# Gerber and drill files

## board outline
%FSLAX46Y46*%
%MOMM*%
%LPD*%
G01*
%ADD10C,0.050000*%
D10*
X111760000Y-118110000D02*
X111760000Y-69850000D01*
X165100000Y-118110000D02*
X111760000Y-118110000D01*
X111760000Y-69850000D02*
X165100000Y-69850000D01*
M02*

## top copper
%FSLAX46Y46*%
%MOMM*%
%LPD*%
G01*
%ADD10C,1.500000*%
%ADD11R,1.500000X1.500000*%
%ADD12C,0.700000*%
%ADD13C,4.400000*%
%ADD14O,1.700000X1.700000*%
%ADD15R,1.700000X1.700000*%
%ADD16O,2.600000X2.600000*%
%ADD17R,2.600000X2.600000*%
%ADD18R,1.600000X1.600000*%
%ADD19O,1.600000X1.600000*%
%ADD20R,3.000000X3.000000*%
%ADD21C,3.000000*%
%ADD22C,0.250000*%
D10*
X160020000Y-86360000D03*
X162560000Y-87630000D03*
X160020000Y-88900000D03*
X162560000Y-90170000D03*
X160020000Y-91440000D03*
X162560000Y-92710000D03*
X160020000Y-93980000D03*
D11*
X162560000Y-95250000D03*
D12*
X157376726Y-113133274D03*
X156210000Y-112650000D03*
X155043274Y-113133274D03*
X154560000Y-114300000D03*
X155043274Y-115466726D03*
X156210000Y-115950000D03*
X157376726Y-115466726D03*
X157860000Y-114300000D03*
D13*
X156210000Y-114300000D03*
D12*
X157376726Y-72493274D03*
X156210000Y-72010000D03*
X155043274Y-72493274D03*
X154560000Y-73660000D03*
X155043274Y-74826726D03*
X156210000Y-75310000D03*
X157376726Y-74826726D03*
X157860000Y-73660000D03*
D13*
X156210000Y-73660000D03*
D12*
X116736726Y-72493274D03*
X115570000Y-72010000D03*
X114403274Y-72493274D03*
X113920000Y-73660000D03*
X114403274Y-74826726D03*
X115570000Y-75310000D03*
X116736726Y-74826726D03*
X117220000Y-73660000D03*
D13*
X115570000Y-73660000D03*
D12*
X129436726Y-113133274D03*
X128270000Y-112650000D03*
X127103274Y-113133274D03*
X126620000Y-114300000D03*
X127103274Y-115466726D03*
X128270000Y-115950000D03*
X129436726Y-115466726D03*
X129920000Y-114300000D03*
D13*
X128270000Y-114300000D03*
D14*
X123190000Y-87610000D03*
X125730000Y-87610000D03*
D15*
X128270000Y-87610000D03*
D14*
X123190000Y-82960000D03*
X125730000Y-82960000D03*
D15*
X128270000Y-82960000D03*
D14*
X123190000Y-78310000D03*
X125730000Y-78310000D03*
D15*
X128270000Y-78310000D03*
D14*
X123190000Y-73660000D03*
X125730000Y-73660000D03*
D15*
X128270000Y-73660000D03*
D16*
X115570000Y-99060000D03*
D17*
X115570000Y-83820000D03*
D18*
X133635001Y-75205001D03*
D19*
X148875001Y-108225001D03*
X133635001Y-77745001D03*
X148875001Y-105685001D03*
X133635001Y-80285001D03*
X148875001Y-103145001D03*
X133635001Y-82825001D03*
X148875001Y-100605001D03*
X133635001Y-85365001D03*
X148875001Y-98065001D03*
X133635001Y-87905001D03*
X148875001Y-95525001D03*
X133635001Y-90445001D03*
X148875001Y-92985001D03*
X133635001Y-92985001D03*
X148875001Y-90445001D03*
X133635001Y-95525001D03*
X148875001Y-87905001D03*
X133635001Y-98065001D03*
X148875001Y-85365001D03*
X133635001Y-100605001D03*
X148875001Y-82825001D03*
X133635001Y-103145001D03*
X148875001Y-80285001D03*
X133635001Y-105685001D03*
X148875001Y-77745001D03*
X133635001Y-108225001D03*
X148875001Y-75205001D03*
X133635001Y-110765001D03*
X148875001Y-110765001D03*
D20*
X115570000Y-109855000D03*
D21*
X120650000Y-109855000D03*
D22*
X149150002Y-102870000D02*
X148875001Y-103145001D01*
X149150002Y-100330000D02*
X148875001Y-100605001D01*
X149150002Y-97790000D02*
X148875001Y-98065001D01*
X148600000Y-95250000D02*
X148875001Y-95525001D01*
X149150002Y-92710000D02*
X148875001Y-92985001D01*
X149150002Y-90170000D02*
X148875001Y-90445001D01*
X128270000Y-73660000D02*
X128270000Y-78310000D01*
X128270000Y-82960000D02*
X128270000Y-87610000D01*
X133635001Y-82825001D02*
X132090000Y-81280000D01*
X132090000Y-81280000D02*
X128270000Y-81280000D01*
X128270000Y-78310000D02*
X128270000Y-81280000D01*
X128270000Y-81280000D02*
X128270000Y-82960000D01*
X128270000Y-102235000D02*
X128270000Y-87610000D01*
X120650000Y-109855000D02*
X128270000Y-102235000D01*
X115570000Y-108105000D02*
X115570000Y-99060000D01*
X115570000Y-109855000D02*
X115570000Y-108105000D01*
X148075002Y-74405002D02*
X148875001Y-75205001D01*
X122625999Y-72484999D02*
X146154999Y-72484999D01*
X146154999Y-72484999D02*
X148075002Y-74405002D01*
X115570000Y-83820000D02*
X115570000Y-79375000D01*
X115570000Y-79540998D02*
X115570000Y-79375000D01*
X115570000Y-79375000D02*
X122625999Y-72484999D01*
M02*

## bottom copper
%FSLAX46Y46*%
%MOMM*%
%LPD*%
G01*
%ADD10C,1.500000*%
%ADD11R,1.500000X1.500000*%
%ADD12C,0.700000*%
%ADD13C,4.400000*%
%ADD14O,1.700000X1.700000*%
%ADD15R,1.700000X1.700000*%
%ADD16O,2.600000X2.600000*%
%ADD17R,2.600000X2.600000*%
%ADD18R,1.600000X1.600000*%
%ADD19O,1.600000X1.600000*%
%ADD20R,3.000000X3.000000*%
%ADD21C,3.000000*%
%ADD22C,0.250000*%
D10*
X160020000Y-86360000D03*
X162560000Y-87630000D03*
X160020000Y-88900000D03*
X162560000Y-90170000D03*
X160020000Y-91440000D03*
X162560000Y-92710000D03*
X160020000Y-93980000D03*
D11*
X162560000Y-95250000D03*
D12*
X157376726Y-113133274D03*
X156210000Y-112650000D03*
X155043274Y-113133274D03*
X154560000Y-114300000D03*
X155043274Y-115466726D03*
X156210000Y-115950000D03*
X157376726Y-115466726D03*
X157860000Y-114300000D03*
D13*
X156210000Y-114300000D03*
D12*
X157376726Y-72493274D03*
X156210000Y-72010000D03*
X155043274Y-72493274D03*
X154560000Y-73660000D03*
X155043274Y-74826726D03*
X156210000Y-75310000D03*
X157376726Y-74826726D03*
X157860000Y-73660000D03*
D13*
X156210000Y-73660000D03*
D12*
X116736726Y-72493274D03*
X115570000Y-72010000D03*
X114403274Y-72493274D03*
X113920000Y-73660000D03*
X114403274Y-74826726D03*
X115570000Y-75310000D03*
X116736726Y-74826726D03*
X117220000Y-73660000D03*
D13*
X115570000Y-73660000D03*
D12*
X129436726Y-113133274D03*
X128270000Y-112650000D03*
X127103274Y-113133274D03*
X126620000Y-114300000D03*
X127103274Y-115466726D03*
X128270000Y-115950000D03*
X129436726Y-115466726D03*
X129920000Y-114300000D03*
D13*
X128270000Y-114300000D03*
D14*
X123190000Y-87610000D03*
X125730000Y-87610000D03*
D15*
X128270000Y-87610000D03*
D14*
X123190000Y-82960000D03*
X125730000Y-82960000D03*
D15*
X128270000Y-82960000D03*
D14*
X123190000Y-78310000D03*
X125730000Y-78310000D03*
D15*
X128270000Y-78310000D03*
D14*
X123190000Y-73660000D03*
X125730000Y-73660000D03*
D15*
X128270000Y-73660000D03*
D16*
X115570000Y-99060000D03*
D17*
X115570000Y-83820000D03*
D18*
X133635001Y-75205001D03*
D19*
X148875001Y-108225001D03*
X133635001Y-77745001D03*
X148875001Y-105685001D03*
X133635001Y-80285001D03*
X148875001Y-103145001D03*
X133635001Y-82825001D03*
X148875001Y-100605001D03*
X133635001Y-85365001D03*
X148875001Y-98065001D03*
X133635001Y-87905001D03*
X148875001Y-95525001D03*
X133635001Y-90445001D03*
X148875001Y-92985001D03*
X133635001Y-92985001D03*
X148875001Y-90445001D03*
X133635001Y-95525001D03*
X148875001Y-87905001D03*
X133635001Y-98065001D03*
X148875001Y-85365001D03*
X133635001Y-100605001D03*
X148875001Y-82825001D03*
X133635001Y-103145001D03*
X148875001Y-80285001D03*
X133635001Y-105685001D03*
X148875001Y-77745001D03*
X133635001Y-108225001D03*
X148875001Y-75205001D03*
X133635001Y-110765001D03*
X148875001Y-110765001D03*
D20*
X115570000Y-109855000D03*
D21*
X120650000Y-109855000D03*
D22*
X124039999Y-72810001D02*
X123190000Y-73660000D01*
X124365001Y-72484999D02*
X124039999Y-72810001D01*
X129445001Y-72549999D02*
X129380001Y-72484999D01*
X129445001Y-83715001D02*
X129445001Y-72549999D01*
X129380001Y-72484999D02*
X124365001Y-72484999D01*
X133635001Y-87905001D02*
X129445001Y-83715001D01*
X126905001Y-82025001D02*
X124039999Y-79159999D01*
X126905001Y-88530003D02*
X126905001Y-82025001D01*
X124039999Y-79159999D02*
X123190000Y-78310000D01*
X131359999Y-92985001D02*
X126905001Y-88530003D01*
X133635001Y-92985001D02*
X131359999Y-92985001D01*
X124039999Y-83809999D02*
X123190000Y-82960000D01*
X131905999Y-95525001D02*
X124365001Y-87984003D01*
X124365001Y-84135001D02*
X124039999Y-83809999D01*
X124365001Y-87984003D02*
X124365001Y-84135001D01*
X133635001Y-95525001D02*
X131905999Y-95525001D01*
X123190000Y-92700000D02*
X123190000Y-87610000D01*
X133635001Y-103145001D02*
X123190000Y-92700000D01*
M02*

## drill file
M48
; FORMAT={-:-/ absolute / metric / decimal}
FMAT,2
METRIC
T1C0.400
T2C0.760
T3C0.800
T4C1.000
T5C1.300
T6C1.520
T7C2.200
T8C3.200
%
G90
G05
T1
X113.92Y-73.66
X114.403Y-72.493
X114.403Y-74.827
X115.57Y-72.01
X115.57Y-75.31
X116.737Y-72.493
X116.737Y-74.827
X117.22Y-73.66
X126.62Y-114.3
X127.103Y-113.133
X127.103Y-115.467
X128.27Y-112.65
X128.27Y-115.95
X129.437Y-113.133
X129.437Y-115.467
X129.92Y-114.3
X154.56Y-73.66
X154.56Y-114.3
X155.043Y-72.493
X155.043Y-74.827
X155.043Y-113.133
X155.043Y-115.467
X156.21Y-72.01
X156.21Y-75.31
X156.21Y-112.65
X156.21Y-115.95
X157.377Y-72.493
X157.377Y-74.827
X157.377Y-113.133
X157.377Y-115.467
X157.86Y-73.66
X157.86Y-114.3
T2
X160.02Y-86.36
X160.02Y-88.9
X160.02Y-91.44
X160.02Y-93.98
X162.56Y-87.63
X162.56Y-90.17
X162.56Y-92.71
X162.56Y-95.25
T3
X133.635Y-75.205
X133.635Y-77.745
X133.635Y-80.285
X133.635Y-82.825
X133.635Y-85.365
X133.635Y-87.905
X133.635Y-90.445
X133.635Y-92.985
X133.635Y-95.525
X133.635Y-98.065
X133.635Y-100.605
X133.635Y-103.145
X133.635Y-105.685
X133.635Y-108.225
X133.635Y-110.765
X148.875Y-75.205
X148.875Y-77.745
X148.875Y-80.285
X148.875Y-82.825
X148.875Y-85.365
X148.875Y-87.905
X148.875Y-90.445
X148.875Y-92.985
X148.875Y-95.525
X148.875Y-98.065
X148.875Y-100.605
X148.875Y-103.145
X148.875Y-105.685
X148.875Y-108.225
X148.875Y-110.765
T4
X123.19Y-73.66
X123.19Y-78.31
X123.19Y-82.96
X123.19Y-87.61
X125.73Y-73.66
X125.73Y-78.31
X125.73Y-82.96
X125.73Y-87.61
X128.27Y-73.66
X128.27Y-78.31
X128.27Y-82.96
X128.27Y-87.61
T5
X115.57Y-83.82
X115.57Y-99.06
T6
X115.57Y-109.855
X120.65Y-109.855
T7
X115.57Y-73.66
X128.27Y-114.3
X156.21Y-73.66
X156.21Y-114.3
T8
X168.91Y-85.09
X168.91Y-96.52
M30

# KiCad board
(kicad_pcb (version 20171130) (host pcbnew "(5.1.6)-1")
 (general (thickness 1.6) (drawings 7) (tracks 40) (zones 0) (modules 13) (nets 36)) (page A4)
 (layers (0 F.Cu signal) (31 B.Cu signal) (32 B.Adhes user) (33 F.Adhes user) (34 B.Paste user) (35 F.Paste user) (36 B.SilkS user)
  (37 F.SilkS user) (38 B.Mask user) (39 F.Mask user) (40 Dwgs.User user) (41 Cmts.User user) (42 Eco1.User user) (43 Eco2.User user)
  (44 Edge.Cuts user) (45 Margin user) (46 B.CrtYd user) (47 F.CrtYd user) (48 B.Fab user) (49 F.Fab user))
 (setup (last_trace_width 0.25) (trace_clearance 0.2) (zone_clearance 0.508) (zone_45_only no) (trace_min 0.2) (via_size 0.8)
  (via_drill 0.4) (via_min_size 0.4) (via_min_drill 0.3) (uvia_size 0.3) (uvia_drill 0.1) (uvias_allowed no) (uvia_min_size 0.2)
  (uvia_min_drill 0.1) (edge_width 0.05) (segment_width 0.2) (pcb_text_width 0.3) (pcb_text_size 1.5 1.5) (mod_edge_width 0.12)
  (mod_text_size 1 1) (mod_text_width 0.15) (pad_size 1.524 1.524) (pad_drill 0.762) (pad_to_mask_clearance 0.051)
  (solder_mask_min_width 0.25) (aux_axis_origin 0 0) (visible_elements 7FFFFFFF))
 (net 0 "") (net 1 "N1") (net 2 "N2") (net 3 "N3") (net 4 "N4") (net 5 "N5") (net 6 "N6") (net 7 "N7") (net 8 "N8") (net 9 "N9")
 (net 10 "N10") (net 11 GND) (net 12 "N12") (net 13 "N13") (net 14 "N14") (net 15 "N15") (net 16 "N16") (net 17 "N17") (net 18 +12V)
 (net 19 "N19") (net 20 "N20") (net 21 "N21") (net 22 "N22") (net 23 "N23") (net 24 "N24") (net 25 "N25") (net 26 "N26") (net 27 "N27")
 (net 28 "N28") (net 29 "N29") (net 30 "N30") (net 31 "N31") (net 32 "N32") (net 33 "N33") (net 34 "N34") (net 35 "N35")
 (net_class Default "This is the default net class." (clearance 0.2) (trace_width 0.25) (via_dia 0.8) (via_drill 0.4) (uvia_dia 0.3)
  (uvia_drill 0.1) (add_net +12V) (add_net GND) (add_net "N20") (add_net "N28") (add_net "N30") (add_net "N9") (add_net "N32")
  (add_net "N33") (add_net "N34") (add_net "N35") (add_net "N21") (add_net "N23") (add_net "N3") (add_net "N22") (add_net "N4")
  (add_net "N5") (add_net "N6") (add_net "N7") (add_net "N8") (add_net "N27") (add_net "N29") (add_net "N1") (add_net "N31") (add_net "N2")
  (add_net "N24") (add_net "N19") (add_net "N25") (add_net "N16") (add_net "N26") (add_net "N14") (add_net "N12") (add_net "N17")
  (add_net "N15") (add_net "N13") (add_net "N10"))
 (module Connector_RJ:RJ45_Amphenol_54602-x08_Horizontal (layer F.Cu) (at 162.56 95.25 90)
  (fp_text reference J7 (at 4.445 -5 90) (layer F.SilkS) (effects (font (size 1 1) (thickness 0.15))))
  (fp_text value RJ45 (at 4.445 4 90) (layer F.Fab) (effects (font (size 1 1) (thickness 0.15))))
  (pad 8 thru_hole circle (at 8.89 -2.54 90) (size 1.5 1.5) (drill 0.76) (layers *.Cu *.Mask) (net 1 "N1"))
  (pad 7 thru_hole circle (at 7.62 0 90) (size 1.5 1.5) (drill 0.76) (layers *.Cu *.Mask) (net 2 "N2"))
  (pad 6 thru_hole circle (at 6.35 -2.54 90) (size 1.5 1.5) (drill 0.76) (layers *.Cu *.Mask) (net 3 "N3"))
  (pad 5 thru_hole circle (at 5.08 0 90) (size 1.5 1.5) (drill 0.76) (layers *.Cu *.Mask) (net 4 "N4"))
  (pad 4 thru_hole circle (at 3.81 -2.54 90) (size 1.5 1.5) (drill 0.76) (layers *.Cu *.Mask) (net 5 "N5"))
  (pad 3 thru_hole circle (at 2.54 0 90) (size 1.5 1.5) (drill 0.76) (layers *.Cu *.Mask) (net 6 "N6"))
  (pad 2 thru_hole circle (at 1.27 -2.54 90) (size 1.5 1.5) (drill 0.76) (layers *.Cu *.Mask) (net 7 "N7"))
  (pad 1 thru_hole rect (at 0 0 90) (size 1.5 1.5) (drill 0.76) (layers *.Cu *.Mask) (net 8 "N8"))
  (pad "" np_thru_hole circle (at -1.27 6.35 90) (size 3.2 3.2) (drill 3.2) (layers *.Cu *.Mask))
  (pad "" np_thru_hole circle (at 10.16 6.35 90) (size 3.2 3.2) (drill 3.2) (layers *.Cu *.Mask)))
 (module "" (layer B.Cu) (at 140.97 92.71 270)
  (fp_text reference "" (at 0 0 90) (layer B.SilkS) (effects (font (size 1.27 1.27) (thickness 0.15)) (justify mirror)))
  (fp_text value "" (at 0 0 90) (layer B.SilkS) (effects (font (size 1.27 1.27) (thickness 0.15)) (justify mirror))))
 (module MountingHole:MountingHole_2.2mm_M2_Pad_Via (layer F.Cu) (at 156.21 114.3)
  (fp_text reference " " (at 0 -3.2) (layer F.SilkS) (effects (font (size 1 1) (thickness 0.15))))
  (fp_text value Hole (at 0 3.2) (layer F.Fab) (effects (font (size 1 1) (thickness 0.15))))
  (pad 1 thru_hole circle (at 1.166726 -1.166726) (size 0.7 0.7) (drill 0.4) (layers *.Cu *.Mask))
  (pad 1 thru_hole circle (at 0 -1.65) (size 0.7 0.7) (drill 0.4) (layers *.Cu *.Mask))
  (pad 1 thru_hole circle (at -1.166726 -1.166726) (size 0.7 0.7) (drill 0.4) (layers *.Cu *.Mask))
  (pad 1 thru_hole circle (at -1.65 0) (size 0.7 0.7) (drill 0.4) (layers *.Cu *.Mask))
  (pad 1 thru_hole circle (at -1.166726 1.166726) (size 0.7 0.7) (drill 0.4) (layers *.Cu *.Mask))
  (pad 1 thru_hole circle (at 0 1.65) (size 0.7 0.7) (drill 0.4) (layers *.Cu *.Mask))
  (pad 1 thru_hole circle (at 1.166726 1.166726) (size 0.7 0.7) (drill 0.4) (layers *.Cu *.Mask))
  (pad 1 thru_hole circle (at 1.65 0) (size 0.7 0.7) (drill 0.4) (layers *.Cu *.Mask))
  (pad 1 thru_hole circle (at 0 0) (size 4.4 4.4) (drill 2.2) (layers *.Cu *.Mask)))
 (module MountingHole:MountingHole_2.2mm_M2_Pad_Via (layer F.Cu) (at 156.21 73.66)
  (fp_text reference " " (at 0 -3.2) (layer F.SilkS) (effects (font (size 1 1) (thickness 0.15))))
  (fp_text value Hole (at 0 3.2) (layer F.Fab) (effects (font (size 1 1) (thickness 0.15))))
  (pad 1 thru_hole circle (at 1.166726 -1.166726) (size 0.7 0.7) (drill 0.4) (layers *.Cu *.Mask))
  (pad 1 thru_hole circle (at 0 -1.65) (size 0.7 0.7) (drill 0.4) (layers *.Cu *.Mask))
  (pad 1 thru_hole circle (at -1.166726 -1.166726) (size 0.7 0.7) (drill 0.4) (layers *.Cu *.Mask))
  (pad 1 thru_hole circle (at -1.65 0) (size 0.7 0.7) (drill 0.4) (layers *.Cu *.Mask))
  (pad 1 thru_hole circle (at -1.166726 1.166726) (size 0.7 0.7) (drill 0.4) (layers *.Cu *.Mask))
  (pad 1 thru_hole circle (at 0 1.65) (size 0.7 0.7) (drill 0.4) (layers *.Cu *.Mask))
  (pad 1 thru_hole circle (at 1.166726 1.166726) (size 0.7 0.7) (drill 0.4) (layers *.Cu *.Mask))
  (pad 1 thru_hole circle (at 1.65 0) (size 0.7 0.7) (drill 0.4) (layers *.Cu *.Mask))
  (pad 1 thru_hole circle (at 0 0) (size 4.4 4.4) (drill 2.2) (layers *.Cu *.Mask)))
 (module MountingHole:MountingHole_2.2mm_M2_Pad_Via (layer F.Cu) (at 115.57 73.66)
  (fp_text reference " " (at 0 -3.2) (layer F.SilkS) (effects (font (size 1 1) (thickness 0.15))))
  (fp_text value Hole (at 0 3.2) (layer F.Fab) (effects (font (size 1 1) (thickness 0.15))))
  (pad 1 thru_hole circle (at 1.166726 -1.166726) (size 0.7 0.7) (drill 0.4) (layers *.Cu *.Mask))
  (pad 1 thru_hole circle (at 0 -1.65) (size 0.7 0.7) (drill 0.4) (layers *.Cu *.Mask))
  (pad 1 thru_hole circle (at -1.166726 -1.166726) (size 0.7 0.7) (drill 0.4) (layers *.Cu *.Mask))
  (pad 1 thru_hole circle (at -1.65 0) (size 0.7 0.7) (drill 0.4) (layers *.Cu *.Mask))
  (pad 1 thru_hole circle (at -1.166726 1.166726) (size 0.7 0.7) (drill 0.4) (layers *.Cu *.Mask))
  (pad 1 thru_hole circle (at 0 1.65) (size 0.7 0.7) (drill 0.4) (layers *.Cu *.Mask))
  (pad 1 thru_hole circle (at 1.166726 1.166726) (size 0.7 0.7) (drill 0.4) (layers *.Cu *.Mask))
  (pad 1 thru_hole circle (at 1.65 0) (size 0.7 0.7) (drill 0.4) (layers *.Cu *.Mask))
  (pad 1 thru_hole circle (at 0 0) (size 4.4 4.4) (drill 2.2) (layers *.Cu *.Mask)))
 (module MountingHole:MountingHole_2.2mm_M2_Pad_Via (layer F.Cu) (at 128.27 114.3)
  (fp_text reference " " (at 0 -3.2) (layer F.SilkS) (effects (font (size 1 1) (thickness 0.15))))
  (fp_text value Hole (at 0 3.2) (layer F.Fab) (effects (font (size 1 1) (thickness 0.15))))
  (pad 1 thru_hole circle (at 1.166726 -1.166726) (size 0.7 0.7) (drill 0.4) (layers *.Cu *.Mask))
  (pad 1 thru_hole circle (at 0 -1.65) (size 0.7 0.7) (drill 0.4) (layers *.Cu *.Mask))
  (pad 1 thru_hole circle (at -1.166726 -1.166726) (size 0.7 0.7) (drill 0.4) (layers *.Cu *.Mask))
  (pad 1 thru_hole circle (at -1.65 0) (size 0.7 0.7) (drill 0.4) (layers *.Cu *.Mask))
  (pad 1 thru_hole circle (at -1.166726 1.166726) (size 0.7 0.7) (drill 0.4) (layers *.Cu *.Mask))
  (pad 1 thru_hole circle (at 0 1.65) (size 0.7 0.7) (drill 0.4) (layers *.Cu *.Mask))
  (pad 1 thru_hole circle (at 1.166726 1.166726) (size 0.7 0.7) (drill 0.4) (layers *.Cu *.Mask))
  (pad 1 thru_hole circle (at 1.65 0) (size 0.7 0.7) (drill 0.4) (layers *.Cu *.Mask))
  (pad 1 thru_hole circle (at 0 0) (size 4.4 4.4) (drill 2.2) (layers *.Cu *.Mask)))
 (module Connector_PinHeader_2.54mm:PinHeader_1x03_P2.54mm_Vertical (layer F.Cu) (at 128.27 87.61 270)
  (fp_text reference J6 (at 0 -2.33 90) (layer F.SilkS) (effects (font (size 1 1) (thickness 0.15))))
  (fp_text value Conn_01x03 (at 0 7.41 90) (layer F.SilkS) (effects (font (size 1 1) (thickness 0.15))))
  (pad 3 thru_hole oval (at 0 5.08 270) (size 1.7 1.7) (drill 1) (layers *.Cu *.Mask) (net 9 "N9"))
  (pad 2 thru_hole oval (at 0 2.54 270) (size 1.7 1.7) (drill 1) (layers *.Cu *.Mask) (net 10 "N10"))
  (pad 1 thru_hole rect (at 0 0 270) (size 1.7 1.7) (drill 1) (layers *.Cu *.Mask) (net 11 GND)))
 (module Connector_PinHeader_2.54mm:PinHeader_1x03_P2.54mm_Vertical (layer F.Cu) (at 128.27 82.96 270)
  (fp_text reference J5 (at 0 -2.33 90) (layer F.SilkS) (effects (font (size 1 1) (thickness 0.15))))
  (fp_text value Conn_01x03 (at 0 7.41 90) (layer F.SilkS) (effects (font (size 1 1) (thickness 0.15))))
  (pad 3 thru_hole oval (at 0 5.08 270) (size 1.7 1.7) (drill 1) (layers *.Cu *.Mask) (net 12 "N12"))
  (pad 2 thru_hole oval (at 0 2.54 270) (size 1.7 1.7) (drill 1) (layers *.Cu *.Mask) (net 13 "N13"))
  (pad 1 thru_hole rect (at 0 0 270) (size 1.7 1.7) (drill 1) (layers *.Cu *.Mask) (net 11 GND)))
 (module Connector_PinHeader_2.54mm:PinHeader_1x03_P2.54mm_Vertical (layer F.Cu) (at 128.27 78.31 270)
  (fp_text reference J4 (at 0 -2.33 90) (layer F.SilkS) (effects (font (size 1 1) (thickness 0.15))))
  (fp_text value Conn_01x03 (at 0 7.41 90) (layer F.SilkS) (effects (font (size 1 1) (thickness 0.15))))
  (pad 3 thru_hole oval (at 0 5.08 270) (size 1.7 1.7) (drill 1) (layers *.Cu *.Mask) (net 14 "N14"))
  (pad 2 thru_hole oval (at 0 2.54 270) (size 1.7 1.7) (drill 1) (layers *.Cu *.Mask) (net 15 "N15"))
  (pad 1 thru_hole rect (at 0 0 270) (size 1.7 1.7) (drill 1) (layers *.Cu *.Mask) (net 11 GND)))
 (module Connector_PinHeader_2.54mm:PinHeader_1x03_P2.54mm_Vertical (layer F.Cu) (at 128.27 73.66 270)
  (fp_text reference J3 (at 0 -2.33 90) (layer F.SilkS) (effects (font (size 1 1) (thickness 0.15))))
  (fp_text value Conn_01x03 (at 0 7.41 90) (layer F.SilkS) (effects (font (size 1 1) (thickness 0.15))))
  (pad 3 thru_hole oval (at 0 5.08 270) (size 1.7 1.7) (drill 1) (layers *.Cu *.Mask) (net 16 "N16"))
  (pad 2 thru_hole oval (at 0 2.54 270) (size 1.7 1.7) (drill 1) (layers *.Cu *.Mask) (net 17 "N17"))
  (pad 1 thru_hole rect (at 0 0 270) (size 1.7 1.7) (drill 1) (layers *.Cu *.Mask) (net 11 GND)))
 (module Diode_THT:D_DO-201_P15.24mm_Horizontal (layer F.Cu) (at 115.57 83.82 270)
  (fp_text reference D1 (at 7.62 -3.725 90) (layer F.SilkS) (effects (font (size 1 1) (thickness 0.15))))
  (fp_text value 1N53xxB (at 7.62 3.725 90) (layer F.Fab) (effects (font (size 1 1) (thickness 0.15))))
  (pad 2 thru_hole oval (at 15.24 0 270) (size 2.6 2.6) (drill 1.3) (layers *.Cu *.Mask) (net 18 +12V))
  (pad 1 thru_hole rect (at 0 0 270) (size 2.6 2.6) (drill 1.3) (layers *.Cu *.Mask) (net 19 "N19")))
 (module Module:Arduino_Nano (layer F.Cu) (at 133.635001 75.205001)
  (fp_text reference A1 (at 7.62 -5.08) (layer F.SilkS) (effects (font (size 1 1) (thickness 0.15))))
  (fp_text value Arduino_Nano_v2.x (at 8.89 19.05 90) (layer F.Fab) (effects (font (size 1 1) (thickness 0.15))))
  (pad 1 thru_hole rect (at 0 0) (size 1.6 1.6) (drill 0.8) (layers *.Cu *.Mask) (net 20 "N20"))
  (pad 17 thru_hole oval (at 15.24 33.02) (size 1.6 1.6) (drill 0.8) (layers *.Cu *.Mask) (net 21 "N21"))
  (pad 2 thru_hole oval (at 0 2.54) (size 1.6 1.6) (drill 0.8) (layers *.Cu *.Mask) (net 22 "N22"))
  (pad 18 thru_hole oval (at 15.24 30.48) (size 1.6 1.6) (drill 0.8) (layers *.Cu *.Mask) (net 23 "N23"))
  (pad 3 thru_hole oval (at 0 5.08) (size 1.6 1.6) (drill 0.8) (layers *.Cu *.Mask) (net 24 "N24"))
  (pad 19 thru_hole oval (at 15.24 27.94) (size 1.6 1.6) (drill 0.8) (layers *.Cu *.Mask) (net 3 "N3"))
  (pad 4 thru_hole oval (at 0 7.62) (size 1.6 1.6) (drill 0.8) (layers *.Cu *.Mask) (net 11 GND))
  (pad 20 thru_hole oval (at 15.24 25.4) (size 1.6 1.6) (drill 0.8) (layers *.Cu *.Mask) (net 4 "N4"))
  (pad 5 thru_hole oval (at 0 10.16) (size 1.6 1.6) (drill 0.8) (layers *.Cu *.Mask) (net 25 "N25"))
  (pad 21 thru_hole oval (at 15.24 22.86) (size 1.6 1.6) (drill 0.8) (layers *.Cu *.Mask) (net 5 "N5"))
  (pad 6 thru_hole oval (at 0 12.7) (size 1.6 1.6) (drill 0.8) (layers *.Cu *.Mask) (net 16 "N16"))
  (pad 22 thru_hole oval (at 15.24 20.32) (size 1.6 1.6) (drill 0.8) (layers *.Cu *.Mask) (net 6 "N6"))
  (pad 7 thru_hole oval (at 0 15.24) (size 1.6 1.6) (drill 0.8) (layers *.Cu *.Mask) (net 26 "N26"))
  (pad 23 thru_hole oval (at 15.24 17.78) (size 1.6 1.6) (drill 0.8) (layers *.Cu *.Mask) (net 7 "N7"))
  (pad 8 thru_hole oval (at 0 17.78) (size 1.6 1.6) (drill 0.8) (layers *.Cu *.Mask) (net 14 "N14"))
  (pad 24 thru_hole oval (at 15.24 15.24) (size 1.6 1.6) (drill 0.8) (layers *.Cu *.Mask) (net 8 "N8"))
  (pad 9 thru_hole oval (at 0 20.32) (size 1.6 1.6) (drill 0.8) (layers *.Cu *.Mask) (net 12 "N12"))
  (pad 25 thru_hole oval (at 15.24 12.7) (size 1.6 1.6) (drill 0.8) (layers *.Cu *.Mask) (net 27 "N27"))
  (pad 10 thru_hole oval (at 0 22.86) (size 1.6 1.6) (drill 0.8) (layers *.Cu *.Mask) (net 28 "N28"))
  (pad 26 thru_hole oval (at 15.24 10.16) (size 1.6 1.6) (drill 0.8) (layers *.Cu *.Mask) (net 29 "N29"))
  (pad 11 thru_hole oval (at 0 25.4) (size 1.6 1.6) (drill 0.8) (layers *.Cu *.Mask) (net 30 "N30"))
  (pad 27 thru_hole oval (at 15.24 7.62) (size 1.6 1.6) (drill 0.8) (layers *.Cu *.Mask) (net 1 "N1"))
  (pad 12 thru_hole oval (at 0 27.94) (size 1.6 1.6) (drill 0.8) (layers *.Cu *.Mask) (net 9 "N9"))
  (pad 28 thru_hole oval (at 15.24 5.08) (size 1.6 1.6) (drill 0.8) (layers *.Cu *.Mask) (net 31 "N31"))
  (pad 13 thru_hole oval (at 0 30.48) (size 1.6 1.6) (drill 0.8) (layers *.Cu *.Mask) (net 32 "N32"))
  (pad 29 thru_hole oval (at 15.24 2.54) (size 1.6 1.6) (drill 0.8) (layers *.Cu *.Mask) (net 2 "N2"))
  (pad 14 thru_hole oval (at 0 33.02) (size 1.6 1.6) (drill 0.8) (layers *.Cu *.Mask) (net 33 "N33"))
  (pad 30 thru_hole oval (at 15.24 0) (size 1.6 1.6) (drill 0.8) (layers *.Cu *.Mask) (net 19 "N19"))
  (pad 15 thru_hole oval (at 0 35.56) (size 1.6 1.6) (drill 0.8) (layers *.Cu *.Mask) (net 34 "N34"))
  (pad 16 thru_hole oval (at 15.24 35.56) (size 1.6 1.6) (drill 0.8) (layers *.Cu *.Mask) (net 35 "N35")))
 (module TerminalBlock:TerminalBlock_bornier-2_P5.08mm (layer F.Cu) (at 115.57 109.855)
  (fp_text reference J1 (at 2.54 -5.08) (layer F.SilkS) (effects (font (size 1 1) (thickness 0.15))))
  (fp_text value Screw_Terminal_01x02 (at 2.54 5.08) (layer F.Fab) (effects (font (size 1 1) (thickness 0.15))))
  (pad 1 thru_hole rect (at 0 0) (size 3 3) (drill 1.52) (layers *.Cu *.Mask) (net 18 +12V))
  (pad 2 thru_hole circle (at 5.08 0) (size 3 3) (drill 1.52) (layers *.Cu *.Mask) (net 11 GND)))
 (gr_line (start 111.76 118.11) (end 111.76 69.85) (layer Edge.Cuts) (width 0.05))
 (gr_line (start 165.1 118.11) (end 111.76 118.11) (layer Edge.Cuts) (width 0.05))
 (gr_line (start 111.76 69.85) (end 165.1 69.85) (layer Edge.Cuts) (width 0.05))
 (segment (start 149.150002 102.87) (end 148.875001 103.145001) (width 0.25) (layer F.Cu) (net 3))
 (segment (start 149.150002 100.33) (end 148.875001 100.605001) (width 0.25) (layer F.Cu) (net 4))
 (segment (start 149.150002 97.79) (end 148.875001 98.065001) (width 0.25) (layer F.Cu) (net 5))
 (segment (start 124.039999 72.810001) (end 123.19 73.66) (width 0.25) (layer B.Cu) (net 16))
 (segment (start 124.365001 72.484999) (end 124.039999 72.810001) (width 0.25) (layer B.Cu) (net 16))
 (segment (start 129.445001 72.549999) (end 129.380001 72.484999) (width 0.25) (layer B.Cu) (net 16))
 (segment (start 129.445001 83.715001) (end 129.445001 72.549999) (width 0.25) (layer B.Cu) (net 16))
 (segment (start 129.380001 72.484999) (end 124.365001 72.484999) (width 0.25) (layer B.Cu) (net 16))
 (segment (start 133.635001 87.905001) (end 129.445001 83.715001) (width 0.25) (layer B.Cu) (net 16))
 (segment (start 148.6 95.25) (end 148.875001 95.525001) (width 0.25) (layer F.Cu) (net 6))
 (segment (start 149.150002 92.71) (end 148.875001 92.985001) (width 0.25) (layer F.Cu) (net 7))
 (segment (start 126.905001 82.025001) (end 124.039999 79.159999) (width 0.25) (layer B.Cu) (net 14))
 (segment (start 126.905001 88.530003) (end 126.905001 82.025001) (width 0.25) (layer B.Cu) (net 14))
 (segment (start 124.039999 79.159999) (end 123.19 78.31) (width 0.25) (layer B.Cu) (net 14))
 (segment (start 131.359999 92.985001) (end 126.905001 88.530003) (width 0.25) (layer B.Cu) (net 14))
 (segment (start 133.635001 92.985001) (end 131.359999 92.985001) (width 0.25) (layer B.Cu) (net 14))
 (segment (start 149.150002 90.17) (end 148.875001 90.445001) (width 0.25) (layer F.Cu) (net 8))
 (segment (start 124.039999 83.809999) (end 123.19 82.96) (width 0.25) (layer B.Cu) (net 12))
 (segment (start 131.905999 95.525001) (end 124.365001 87.984003) (width 0.25) (layer B.Cu) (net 12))
 (segment (start 124.365001 84.135001) (end 124.039999 83.809999) (width 0.25) (layer B.Cu) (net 12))
 (segment (start 124.365001 87.984003) (end 124.365001 84.135001) (width 0.25) (layer B.Cu) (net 12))
 (segment (start 133.635001 95.525001) (end 131.905999 95.525001) (width 0.25) (layer B.Cu) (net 12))
 (segment (start 123.19 92.7) (end 123.19 87.61) (width 0.25) (layer B.Cu) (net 9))
 (segment (start 133.635001 103.145001) (end 123.19 92.7) (width 0.25) (layer B.Cu) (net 9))
 (segment (start 128.27 73.66) (end 128.27 78.31) (width 0.25) (layer F.Cu) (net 11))
 (segment (start 128.27 82.96) (end 128.27 87.61) (width 0.25) (layer F.Cu) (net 11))
 (segment (start 133.635001 82.825001) (end 132.09 81.28) (width 0.25) (layer F.Cu) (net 11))
 (segment (start 132.09 81.28) (end 128.27 81.28) (width 0.25) (layer F.Cu) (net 11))
 (segment (start 128.27 78.31) (end 128.27 81.28) (width 0.25) (layer F.Cu) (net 11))
 (segment (start 128.27 81.28) (end 128.27 82.96) (width 0.25) (layer F.Cu) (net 11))
 (segment (start 128.27 102.235) (end 128.27 87.61) (width 0.25) (layer F.Cu) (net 11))
 (segment (start 120.65 109.855) (end 128.27 102.235) (width 0.25) (layer F.Cu) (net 11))
 (segment (start 115.57 108.105) (end 115.57 99.06) (width 0.25) (layer F.Cu) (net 18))
 (segment (start 115.57 109.855) (end 115.57 108.105) (width 0.25) (layer F.Cu) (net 18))
 (segment (start 148.075002 74.405002) (end 148.875001 75.205001) (width 0.25) (layer F.Cu) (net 19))
 (segment (start 122.625999 72.484999) (end 146.154999 72.484999) (width 0.25) (layer F.Cu) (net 19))
 (segment (start 146.154999 72.484999) (end 148.075002 74.405002) (width 0.25) (layer F.Cu) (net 19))
 (segment (start 115.57 83.82) (end 115.57 79.375) (width 0.25) (layer F.Cu) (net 19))
 (segment (start 115.57 79.540998) (end 115.57 79.375) (width 0.25) (layer F.Cu) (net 19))
 (segment (start 115.57 79.375) (end 122.625999 72.484999) (width 0.25) (layer F.Cu) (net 19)))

